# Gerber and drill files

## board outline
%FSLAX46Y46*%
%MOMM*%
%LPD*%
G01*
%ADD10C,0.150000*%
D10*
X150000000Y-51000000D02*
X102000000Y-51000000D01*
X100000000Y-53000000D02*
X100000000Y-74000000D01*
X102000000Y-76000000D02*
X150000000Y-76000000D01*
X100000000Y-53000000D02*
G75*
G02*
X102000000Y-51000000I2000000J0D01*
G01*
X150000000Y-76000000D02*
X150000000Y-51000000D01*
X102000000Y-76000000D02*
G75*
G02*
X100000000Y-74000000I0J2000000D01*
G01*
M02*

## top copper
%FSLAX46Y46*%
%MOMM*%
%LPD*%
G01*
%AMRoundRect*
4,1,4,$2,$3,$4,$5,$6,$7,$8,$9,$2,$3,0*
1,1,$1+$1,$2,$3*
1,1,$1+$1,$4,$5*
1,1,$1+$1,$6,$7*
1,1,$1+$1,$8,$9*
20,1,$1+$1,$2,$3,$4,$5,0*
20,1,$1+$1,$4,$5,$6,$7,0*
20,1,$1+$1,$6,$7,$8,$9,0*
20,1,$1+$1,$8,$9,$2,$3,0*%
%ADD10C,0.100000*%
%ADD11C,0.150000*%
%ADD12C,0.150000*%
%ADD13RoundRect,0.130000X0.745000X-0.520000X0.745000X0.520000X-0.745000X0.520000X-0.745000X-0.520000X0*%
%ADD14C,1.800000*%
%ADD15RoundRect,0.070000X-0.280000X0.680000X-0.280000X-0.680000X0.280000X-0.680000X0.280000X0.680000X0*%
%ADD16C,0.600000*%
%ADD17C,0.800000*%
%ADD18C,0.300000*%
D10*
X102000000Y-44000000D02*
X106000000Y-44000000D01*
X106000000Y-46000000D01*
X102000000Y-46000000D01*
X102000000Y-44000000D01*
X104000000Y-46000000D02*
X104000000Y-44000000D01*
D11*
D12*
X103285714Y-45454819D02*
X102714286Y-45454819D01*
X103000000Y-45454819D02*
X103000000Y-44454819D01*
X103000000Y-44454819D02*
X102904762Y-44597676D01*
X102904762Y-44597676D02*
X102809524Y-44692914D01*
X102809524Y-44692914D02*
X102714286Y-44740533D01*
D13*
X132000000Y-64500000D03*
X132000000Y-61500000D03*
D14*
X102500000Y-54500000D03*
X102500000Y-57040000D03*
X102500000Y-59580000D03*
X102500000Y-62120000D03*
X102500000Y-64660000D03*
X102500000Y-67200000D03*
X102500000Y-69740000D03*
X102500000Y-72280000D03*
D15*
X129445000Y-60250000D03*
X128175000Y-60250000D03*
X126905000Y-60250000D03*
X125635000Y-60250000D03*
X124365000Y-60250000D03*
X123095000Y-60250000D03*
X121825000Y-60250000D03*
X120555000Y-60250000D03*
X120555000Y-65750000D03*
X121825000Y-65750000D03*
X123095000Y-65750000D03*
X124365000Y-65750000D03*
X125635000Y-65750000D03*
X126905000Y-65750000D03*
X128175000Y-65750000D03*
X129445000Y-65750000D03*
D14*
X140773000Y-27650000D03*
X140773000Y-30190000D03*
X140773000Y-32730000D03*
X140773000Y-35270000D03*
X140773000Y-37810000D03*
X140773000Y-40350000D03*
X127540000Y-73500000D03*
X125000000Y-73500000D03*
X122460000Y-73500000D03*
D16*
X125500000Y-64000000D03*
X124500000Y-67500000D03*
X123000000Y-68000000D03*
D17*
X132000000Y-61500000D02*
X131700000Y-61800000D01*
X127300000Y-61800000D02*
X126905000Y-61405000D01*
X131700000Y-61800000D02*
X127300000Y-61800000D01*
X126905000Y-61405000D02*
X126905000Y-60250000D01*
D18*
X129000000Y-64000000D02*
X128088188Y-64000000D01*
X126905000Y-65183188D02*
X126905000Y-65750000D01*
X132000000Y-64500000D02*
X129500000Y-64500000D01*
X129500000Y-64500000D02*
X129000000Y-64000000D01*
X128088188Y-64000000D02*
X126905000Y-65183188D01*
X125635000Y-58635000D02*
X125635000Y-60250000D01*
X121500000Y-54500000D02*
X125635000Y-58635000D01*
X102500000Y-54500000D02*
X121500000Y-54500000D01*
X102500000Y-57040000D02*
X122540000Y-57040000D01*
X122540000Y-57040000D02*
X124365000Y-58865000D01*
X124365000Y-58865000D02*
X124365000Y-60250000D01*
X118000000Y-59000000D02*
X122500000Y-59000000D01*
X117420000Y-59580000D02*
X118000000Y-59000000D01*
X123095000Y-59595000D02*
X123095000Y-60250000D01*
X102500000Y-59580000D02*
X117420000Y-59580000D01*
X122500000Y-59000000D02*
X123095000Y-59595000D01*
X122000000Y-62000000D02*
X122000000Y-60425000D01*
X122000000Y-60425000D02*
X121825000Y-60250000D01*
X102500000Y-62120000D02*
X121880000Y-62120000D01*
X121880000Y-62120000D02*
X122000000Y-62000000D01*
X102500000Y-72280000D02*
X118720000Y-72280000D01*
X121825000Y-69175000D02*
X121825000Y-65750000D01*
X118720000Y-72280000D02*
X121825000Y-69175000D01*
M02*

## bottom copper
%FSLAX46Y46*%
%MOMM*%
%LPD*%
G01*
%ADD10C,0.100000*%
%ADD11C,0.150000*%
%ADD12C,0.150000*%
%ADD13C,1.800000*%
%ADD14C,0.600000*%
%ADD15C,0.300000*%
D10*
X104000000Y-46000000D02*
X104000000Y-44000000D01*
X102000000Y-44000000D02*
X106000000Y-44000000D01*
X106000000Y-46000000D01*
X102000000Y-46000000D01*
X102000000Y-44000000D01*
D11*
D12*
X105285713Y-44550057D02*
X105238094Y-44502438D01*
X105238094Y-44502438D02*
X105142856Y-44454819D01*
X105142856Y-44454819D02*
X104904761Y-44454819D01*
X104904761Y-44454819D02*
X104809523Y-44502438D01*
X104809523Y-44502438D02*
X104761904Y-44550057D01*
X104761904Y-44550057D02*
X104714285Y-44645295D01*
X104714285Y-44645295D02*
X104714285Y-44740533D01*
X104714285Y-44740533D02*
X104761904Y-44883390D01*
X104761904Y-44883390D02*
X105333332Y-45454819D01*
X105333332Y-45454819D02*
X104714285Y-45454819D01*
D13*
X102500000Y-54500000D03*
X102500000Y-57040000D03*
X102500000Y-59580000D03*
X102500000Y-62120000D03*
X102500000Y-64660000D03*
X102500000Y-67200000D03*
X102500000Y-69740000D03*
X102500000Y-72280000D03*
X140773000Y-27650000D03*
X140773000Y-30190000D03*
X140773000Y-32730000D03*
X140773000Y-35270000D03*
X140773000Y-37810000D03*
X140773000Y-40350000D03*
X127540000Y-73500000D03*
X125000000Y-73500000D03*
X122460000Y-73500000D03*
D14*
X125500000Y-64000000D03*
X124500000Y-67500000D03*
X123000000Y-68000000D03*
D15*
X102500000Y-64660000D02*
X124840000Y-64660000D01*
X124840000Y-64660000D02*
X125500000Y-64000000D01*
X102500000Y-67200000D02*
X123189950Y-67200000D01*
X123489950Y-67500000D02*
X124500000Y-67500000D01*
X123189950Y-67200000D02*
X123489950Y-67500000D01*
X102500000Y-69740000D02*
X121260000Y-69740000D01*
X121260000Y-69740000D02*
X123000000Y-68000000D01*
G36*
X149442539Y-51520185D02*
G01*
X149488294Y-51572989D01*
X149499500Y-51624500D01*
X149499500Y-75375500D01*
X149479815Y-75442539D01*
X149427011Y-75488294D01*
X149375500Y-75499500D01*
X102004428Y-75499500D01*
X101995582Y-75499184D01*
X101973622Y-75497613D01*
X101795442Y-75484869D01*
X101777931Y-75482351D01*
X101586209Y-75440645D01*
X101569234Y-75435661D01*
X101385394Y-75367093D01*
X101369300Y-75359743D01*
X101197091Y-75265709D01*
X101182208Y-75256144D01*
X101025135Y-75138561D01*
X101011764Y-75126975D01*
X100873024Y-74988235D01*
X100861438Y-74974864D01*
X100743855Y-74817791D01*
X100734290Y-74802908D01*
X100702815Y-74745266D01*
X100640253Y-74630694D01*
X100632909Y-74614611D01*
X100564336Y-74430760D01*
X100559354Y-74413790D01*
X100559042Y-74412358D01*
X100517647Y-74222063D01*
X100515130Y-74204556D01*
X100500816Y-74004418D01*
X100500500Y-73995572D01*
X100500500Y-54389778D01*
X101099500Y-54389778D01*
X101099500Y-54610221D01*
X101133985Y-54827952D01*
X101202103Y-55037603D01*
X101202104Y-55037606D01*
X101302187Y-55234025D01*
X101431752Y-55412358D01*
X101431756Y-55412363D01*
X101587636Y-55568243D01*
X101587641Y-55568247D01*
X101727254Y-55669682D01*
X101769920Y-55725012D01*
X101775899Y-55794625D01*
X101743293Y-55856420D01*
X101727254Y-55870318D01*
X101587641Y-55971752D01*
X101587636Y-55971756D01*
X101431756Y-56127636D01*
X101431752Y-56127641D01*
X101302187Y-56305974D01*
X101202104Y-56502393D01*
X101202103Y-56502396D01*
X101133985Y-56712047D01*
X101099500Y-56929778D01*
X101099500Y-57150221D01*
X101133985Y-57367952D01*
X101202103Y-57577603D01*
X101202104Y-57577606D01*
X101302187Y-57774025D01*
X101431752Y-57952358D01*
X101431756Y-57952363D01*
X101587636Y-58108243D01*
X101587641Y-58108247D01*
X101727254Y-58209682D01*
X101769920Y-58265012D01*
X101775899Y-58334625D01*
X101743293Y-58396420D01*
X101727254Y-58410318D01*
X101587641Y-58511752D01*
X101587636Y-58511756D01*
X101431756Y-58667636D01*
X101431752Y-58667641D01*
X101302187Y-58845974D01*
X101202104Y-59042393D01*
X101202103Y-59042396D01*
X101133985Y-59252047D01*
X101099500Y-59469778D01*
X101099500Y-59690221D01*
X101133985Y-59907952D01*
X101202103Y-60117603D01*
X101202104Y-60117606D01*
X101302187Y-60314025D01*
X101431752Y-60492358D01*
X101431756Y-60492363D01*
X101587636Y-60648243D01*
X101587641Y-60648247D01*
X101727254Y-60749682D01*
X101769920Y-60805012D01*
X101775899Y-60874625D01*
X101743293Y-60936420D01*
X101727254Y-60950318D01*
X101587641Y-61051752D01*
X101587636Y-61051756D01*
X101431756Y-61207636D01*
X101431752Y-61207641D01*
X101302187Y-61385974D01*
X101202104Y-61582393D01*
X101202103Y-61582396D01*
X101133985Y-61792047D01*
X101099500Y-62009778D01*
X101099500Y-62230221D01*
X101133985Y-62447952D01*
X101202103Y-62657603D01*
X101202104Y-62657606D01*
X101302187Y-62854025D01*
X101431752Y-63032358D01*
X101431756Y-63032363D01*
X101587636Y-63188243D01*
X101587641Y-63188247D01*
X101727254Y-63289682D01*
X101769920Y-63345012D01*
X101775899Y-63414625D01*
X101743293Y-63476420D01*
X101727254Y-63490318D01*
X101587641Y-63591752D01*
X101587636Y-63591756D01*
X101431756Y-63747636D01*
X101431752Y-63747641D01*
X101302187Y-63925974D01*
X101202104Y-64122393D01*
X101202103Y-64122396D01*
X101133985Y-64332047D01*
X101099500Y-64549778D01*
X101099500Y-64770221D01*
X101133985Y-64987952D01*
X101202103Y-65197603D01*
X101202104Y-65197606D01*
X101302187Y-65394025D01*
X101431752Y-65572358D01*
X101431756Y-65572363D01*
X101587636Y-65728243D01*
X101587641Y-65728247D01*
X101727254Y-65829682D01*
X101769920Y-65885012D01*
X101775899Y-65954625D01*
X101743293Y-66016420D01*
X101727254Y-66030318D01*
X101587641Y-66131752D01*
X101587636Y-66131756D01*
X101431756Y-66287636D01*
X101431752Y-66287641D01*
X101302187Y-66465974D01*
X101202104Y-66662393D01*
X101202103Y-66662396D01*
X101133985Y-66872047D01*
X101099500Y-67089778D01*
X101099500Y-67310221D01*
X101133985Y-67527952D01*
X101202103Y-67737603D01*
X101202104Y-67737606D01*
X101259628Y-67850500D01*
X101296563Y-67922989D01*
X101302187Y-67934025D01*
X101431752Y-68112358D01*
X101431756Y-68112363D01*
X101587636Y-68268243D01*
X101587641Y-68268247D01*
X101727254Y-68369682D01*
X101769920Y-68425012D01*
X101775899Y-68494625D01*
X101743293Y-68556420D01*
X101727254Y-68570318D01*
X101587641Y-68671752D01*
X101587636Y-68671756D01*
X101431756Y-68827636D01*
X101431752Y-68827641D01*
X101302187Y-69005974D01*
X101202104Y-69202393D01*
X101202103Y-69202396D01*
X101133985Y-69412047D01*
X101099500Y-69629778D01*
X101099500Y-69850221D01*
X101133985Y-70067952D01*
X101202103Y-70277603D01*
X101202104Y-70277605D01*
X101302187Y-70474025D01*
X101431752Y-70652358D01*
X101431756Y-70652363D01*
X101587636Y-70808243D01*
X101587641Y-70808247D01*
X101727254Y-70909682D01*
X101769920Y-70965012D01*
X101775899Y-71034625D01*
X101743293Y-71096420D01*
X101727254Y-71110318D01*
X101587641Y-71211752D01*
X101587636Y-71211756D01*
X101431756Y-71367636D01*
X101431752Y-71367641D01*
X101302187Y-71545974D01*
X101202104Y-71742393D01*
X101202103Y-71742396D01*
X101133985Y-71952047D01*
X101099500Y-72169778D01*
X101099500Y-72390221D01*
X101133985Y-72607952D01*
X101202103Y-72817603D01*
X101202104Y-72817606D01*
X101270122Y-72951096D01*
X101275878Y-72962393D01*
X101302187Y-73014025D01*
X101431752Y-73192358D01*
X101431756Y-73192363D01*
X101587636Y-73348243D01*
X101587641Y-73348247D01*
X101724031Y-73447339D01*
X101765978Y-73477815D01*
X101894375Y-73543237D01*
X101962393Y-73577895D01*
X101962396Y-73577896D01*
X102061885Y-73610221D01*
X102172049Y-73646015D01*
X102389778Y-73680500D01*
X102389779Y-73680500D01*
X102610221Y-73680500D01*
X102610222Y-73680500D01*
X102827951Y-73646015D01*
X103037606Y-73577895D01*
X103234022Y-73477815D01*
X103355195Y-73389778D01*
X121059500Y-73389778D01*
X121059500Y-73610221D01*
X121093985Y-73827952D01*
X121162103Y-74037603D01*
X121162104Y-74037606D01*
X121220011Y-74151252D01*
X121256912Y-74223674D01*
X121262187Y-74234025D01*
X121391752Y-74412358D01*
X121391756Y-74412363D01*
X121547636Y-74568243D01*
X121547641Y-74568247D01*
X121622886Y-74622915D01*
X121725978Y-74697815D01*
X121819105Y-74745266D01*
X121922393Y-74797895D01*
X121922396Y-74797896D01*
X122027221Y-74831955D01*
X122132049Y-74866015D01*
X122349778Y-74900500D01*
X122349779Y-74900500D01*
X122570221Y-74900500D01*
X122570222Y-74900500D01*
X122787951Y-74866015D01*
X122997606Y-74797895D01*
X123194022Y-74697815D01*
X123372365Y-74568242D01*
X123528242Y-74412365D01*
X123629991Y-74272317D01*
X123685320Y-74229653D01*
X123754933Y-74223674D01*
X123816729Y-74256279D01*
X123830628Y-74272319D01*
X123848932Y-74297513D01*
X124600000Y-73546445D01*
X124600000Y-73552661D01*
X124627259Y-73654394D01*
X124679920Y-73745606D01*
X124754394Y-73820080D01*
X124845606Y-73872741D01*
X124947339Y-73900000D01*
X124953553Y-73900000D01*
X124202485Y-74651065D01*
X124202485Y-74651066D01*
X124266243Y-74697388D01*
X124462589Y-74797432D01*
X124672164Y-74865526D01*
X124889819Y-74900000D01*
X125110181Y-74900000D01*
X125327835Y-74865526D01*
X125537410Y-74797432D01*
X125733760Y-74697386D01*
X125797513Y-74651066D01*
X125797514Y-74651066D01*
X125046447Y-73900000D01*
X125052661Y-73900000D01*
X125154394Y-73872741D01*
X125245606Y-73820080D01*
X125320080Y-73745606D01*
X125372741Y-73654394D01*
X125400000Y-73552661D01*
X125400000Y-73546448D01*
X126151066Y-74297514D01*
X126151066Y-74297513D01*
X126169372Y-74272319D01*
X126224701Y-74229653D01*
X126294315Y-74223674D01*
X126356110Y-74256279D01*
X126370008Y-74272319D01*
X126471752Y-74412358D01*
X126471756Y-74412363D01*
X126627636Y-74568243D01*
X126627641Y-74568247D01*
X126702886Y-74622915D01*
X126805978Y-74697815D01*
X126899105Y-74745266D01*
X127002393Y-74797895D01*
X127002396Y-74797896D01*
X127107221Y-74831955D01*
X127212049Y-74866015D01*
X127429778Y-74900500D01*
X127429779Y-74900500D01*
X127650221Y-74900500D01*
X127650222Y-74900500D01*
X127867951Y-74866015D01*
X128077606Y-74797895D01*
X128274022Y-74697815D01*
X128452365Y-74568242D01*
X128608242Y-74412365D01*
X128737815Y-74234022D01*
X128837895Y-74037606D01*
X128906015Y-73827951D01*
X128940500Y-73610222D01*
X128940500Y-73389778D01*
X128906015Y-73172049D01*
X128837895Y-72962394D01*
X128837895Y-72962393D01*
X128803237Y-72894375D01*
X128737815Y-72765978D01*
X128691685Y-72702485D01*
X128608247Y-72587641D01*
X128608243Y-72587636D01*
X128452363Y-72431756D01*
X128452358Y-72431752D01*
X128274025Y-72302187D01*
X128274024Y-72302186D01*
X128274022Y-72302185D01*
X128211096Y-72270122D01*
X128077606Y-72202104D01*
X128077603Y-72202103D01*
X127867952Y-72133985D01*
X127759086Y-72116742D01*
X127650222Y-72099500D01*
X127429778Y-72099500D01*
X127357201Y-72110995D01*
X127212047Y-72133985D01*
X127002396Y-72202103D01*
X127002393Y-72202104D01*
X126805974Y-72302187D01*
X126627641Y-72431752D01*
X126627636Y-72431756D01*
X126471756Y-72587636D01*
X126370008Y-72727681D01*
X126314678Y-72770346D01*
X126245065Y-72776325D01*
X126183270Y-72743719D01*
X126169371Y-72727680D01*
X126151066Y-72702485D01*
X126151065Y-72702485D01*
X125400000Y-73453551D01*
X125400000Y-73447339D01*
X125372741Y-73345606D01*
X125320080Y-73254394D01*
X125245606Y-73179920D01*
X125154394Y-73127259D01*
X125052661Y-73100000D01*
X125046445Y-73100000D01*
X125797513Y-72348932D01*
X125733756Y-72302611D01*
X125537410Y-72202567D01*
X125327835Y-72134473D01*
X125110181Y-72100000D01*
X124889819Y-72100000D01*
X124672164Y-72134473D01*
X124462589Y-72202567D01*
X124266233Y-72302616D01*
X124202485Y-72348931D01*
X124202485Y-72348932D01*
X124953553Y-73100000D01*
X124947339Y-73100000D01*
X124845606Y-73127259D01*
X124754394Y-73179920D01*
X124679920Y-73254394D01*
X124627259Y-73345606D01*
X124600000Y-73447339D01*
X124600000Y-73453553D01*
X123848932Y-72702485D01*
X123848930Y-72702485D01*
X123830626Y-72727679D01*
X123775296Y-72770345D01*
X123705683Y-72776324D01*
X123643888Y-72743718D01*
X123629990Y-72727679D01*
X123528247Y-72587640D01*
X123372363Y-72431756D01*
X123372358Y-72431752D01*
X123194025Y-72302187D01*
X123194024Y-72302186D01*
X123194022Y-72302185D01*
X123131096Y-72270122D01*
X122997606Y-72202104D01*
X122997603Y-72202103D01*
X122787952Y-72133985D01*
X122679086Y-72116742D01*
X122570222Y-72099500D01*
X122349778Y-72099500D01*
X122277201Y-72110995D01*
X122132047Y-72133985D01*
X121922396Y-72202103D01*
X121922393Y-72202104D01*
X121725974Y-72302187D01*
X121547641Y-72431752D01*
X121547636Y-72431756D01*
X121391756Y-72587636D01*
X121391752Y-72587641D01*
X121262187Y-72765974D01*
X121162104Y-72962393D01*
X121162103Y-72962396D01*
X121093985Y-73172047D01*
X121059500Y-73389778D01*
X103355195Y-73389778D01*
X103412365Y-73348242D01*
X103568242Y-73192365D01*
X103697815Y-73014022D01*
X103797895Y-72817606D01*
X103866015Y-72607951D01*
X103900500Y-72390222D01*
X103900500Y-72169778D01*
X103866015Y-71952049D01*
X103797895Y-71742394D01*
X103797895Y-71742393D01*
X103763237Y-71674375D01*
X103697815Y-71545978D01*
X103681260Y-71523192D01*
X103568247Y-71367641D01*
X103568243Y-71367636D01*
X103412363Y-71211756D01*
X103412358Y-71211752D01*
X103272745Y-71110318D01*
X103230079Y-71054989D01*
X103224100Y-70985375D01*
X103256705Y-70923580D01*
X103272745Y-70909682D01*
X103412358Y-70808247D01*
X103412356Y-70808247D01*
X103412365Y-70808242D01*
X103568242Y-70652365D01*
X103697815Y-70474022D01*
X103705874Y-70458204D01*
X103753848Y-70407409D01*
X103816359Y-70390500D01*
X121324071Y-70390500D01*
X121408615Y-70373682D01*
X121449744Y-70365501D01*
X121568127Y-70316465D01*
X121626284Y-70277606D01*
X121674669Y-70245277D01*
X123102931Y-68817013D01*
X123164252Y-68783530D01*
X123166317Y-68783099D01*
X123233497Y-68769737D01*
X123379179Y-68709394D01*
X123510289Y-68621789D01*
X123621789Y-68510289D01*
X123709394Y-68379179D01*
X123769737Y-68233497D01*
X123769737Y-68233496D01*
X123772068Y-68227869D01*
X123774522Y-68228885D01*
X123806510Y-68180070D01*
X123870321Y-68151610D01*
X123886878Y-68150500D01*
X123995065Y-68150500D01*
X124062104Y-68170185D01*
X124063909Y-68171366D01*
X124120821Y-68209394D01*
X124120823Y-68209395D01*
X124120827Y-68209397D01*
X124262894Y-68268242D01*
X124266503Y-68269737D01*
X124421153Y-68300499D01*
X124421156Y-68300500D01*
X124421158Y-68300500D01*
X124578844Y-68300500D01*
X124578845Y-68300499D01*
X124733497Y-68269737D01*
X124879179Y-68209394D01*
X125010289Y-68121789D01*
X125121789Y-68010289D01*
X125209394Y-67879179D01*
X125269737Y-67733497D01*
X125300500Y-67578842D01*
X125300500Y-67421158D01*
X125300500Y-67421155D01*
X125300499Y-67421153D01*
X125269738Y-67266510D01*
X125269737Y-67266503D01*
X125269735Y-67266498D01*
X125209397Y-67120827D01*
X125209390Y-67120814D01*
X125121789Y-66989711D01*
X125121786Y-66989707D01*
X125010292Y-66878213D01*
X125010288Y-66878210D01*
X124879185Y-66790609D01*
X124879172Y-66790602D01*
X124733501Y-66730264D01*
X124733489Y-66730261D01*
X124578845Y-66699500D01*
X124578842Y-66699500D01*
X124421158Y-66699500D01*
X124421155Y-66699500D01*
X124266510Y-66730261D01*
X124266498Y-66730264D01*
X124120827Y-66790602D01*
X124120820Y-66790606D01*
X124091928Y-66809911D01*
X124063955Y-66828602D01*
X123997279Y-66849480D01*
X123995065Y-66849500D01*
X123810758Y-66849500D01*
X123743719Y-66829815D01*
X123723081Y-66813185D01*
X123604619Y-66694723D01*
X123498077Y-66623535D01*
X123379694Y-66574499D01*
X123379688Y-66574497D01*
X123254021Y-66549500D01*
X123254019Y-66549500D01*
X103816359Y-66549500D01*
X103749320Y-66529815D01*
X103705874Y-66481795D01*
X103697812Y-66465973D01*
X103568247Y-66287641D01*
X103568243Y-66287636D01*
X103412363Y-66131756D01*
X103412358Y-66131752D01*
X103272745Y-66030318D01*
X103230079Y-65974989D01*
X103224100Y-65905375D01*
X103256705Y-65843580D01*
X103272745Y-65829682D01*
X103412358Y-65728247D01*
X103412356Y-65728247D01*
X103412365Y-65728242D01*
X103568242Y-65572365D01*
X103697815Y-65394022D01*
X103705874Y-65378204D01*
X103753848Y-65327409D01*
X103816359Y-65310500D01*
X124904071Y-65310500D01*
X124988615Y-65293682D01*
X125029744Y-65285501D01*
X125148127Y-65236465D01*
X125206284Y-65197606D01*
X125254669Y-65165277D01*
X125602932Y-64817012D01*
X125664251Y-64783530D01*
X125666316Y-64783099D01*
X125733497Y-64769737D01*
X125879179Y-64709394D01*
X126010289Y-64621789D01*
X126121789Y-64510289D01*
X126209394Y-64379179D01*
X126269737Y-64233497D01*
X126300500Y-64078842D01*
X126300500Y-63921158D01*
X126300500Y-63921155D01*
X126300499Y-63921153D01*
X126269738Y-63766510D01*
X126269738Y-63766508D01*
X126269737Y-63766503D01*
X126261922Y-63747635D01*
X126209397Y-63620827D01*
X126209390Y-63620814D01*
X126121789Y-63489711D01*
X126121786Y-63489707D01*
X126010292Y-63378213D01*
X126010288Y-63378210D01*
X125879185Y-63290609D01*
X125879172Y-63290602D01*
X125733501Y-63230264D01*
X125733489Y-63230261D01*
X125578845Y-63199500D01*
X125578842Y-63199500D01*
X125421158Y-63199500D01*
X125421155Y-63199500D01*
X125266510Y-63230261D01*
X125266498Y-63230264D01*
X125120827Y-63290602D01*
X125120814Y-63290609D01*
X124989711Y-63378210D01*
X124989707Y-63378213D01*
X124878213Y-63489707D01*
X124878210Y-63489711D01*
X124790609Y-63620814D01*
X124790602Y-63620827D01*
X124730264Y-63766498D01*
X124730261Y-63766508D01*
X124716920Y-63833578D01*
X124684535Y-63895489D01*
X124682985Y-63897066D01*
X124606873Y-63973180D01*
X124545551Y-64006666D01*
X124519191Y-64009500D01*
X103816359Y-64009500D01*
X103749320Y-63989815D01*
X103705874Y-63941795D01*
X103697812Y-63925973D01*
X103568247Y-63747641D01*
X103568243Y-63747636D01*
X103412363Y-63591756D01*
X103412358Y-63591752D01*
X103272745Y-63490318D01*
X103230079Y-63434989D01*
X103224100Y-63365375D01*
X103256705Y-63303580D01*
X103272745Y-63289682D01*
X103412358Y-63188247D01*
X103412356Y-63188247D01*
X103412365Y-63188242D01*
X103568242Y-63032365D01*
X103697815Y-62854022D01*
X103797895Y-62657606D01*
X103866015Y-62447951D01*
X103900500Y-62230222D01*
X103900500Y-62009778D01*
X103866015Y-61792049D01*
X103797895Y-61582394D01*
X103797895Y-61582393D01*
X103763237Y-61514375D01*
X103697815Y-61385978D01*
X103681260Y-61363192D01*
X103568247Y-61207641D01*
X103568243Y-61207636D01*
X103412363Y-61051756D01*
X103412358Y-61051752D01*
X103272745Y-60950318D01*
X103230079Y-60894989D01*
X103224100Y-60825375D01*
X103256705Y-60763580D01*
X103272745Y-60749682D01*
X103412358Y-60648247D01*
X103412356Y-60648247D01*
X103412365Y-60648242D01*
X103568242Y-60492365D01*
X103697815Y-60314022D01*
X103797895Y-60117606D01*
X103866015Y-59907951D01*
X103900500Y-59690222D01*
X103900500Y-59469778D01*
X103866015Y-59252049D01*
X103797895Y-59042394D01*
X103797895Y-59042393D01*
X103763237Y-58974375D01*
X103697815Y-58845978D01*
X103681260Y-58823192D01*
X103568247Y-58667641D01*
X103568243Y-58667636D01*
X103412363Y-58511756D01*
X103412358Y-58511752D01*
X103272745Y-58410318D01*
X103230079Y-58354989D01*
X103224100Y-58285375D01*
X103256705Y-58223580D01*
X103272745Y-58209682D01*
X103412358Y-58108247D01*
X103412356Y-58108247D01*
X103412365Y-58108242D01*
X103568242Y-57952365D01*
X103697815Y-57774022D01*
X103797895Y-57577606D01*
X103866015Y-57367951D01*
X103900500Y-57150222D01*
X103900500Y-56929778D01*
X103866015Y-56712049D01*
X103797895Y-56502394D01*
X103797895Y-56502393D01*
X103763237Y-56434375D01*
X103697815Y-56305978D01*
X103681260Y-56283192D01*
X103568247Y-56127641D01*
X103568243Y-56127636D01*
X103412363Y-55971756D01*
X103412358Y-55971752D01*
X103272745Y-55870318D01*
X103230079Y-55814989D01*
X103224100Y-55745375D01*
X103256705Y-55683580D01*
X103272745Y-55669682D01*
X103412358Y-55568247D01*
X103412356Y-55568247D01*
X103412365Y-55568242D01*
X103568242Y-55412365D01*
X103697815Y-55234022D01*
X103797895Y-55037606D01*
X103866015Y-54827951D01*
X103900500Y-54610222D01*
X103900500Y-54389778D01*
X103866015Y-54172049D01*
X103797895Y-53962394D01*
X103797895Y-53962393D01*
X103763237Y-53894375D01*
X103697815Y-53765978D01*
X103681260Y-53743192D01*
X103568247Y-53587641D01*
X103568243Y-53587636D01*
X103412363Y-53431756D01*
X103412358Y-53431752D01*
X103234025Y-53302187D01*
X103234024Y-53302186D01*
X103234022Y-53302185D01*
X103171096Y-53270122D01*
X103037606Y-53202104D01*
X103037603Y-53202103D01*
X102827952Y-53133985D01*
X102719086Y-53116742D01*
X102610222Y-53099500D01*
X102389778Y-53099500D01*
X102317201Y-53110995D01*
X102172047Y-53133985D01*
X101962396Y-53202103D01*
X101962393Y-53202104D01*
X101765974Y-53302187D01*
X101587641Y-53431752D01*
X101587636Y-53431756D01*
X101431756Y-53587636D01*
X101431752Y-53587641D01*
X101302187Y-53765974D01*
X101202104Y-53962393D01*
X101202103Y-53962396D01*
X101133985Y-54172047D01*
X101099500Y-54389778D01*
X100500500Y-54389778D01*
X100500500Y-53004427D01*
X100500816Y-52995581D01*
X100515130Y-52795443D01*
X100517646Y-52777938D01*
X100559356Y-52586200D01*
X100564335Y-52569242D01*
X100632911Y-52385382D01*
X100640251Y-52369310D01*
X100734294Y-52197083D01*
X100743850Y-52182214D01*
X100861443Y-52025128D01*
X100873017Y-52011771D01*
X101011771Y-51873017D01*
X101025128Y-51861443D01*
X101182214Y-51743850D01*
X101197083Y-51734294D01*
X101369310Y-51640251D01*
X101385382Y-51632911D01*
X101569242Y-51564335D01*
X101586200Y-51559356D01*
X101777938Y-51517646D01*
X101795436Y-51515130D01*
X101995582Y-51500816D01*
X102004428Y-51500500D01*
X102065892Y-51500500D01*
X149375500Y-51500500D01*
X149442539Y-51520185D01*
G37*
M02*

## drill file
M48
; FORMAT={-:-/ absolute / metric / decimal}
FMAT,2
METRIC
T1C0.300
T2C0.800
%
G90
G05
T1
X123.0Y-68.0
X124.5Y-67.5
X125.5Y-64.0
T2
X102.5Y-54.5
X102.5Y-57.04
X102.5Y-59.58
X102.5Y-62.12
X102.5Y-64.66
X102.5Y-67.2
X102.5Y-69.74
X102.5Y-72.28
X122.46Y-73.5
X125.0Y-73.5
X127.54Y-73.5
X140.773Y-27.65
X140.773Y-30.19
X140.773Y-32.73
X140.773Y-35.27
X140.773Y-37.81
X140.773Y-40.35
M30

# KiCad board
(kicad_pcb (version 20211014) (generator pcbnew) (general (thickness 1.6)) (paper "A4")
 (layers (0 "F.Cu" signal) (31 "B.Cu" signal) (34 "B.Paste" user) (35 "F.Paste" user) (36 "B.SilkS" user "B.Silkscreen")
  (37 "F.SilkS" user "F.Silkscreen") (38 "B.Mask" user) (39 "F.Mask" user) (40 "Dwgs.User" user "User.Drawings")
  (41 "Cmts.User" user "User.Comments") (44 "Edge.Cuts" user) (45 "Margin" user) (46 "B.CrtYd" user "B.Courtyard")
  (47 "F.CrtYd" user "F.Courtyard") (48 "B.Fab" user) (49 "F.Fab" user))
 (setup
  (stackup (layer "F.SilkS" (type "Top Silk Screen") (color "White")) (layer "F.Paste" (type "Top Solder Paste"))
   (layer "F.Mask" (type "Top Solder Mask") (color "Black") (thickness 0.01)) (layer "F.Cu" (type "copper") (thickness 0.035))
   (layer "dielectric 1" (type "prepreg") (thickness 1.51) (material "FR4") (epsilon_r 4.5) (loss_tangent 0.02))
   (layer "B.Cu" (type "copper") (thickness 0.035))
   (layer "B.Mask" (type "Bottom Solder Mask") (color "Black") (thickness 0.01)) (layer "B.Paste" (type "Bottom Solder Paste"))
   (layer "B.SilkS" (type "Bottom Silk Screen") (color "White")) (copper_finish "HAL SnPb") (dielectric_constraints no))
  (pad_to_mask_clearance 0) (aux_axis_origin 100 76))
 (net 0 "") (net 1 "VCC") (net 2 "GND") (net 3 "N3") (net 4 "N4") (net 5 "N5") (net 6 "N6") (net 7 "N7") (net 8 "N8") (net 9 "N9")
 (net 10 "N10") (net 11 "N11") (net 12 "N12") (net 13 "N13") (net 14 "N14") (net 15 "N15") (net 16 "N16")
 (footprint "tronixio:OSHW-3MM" (layer "F.Cu") (at 148 73.5)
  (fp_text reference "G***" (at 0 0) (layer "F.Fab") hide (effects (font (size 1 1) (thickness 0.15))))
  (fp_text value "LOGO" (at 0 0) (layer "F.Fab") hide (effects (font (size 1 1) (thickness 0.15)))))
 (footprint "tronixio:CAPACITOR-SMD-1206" (layer "F.Cu") (at 132 63 90) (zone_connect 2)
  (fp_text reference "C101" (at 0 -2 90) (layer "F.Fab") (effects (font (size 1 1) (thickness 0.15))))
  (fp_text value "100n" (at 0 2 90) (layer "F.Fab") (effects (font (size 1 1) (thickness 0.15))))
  (pad "1" smd roundrect (at -1.5 0 90) (size 1.3 1.75) (layers "F.Cu" "F.Paste" "F.Mask") (roundrect_rratio 0.1) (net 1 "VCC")
   (zone_connect 2))
  (pad "2" smd roundrect (at 1.5 0 90) (size 1.3 1.75) (layers "F.Cu" "F.Paste" "F.Mask") (roundrect_rratio 0.1) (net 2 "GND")
   (zone_connect 2)))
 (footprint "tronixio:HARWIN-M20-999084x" (layer "F.Cu") (at 102.5 54.5)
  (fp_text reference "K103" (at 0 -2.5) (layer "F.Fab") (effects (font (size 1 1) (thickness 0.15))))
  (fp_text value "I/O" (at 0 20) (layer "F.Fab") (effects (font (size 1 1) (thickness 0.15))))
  (pad "1" thru_hole circle locked (at 0 0) (size 1.8 1.8) (drill 0.8) (layers *.Cu *.Mask) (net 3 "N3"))
  (pad "2" thru_hole circle (at 0 2.54) (size 1.8 1.8) (drill 0.8) (layers *.Cu *.Mask) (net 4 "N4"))
  (pad "3" thru_hole circle (at 0 5.08) (size 1.8 1.8) (drill 0.8) (layers *.Cu *.Mask) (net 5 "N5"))
  (pad "4" thru_hole circle (at 0 7.62) (size 1.8 1.8) (drill 0.8) (layers *.Cu *.Mask) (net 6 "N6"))
  (pad "5" thru_hole circle (at 0 10.16) (size 1.8 1.8) (drill 0.8) (layers *.Cu *.Mask) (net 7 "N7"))
  (pad "6" thru_hole circle (at 0 12.7) (size 1.8 1.8) (drill 0.8) (layers *.Cu *.Mask) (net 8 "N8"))
  (pad "7" thru_hole circle (at 0 15.24) (size 1.8 1.8) (drill 0.8) (layers *.Cu *.Mask) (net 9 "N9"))
  (pad "8" thru_hole circle (at 0 17.78) (size 1.8 1.8) (drill 0.8) (layers *.Cu *.Mask) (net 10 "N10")))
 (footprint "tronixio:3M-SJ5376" (layer "F.Cu") (at 166.4 61.25)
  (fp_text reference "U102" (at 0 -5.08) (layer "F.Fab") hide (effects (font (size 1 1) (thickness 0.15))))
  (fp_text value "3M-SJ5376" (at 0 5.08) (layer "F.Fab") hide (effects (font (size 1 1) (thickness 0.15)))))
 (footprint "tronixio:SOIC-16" (layer "F.Cu") (at 125 63 -90)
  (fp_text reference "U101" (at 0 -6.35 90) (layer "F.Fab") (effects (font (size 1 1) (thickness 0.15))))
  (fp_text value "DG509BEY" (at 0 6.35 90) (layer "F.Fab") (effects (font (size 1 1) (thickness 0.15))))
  (pad "1" smd roundrect (at -2.75 -4.445 270) (size 1.5 0.7) (layers "F.Cu" "F.Paste" "F.Mask") (roundrect_rratio 0.1) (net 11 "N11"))
  (pad "2" smd roundrect (at -2.75 -3.175 270) (size 1.5 0.7) (layers "F.Cu" "F.Paste" "F.Mask") (roundrect_rratio 0.1) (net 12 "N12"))
  (pad "3" smd roundrect (at -2.75 -1.905 270) (size 1.5 0.7) (layers "F.Cu" "F.Paste" "F.Mask") (roundrect_rratio 0.1) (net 2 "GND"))
  (pad "4" smd roundrect (at -2.75 -0.635 270) (size 1.5 0.7) (layers "F.Cu" "F.Paste" "F.Mask") (roundrect_rratio 0.1) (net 3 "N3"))
  (pad "5" smd roundrect (at -2.75 0.635 270) (size 1.5 0.7) (layers "F.Cu" "F.Paste" "F.Mask") (roundrect_rratio 0.1) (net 4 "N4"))
  (pad "6" smd roundrect (at -2.75 1.905 270) (size 1.5 0.7) (layers "F.Cu" "F.Paste" "F.Mask") (roundrect_rratio 0.1) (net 5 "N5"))
  (pad "7" smd roundrect (at -2.75 3.175 270) (size 1.5 0.7) (layers "F.Cu" "F.Paste" "F.Mask") (roundrect_rratio 0.1) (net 6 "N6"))
  (pad "8" smd roundrect (at -2.75 4.445 270) (size 1.5 0.7) (layers "F.Cu" "F.Paste" "F.Mask") (roundrect_rratio 0.1) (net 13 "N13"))
  (pad "9" smd roundrect (at 2.75 4.445 270) (size 1.5 0.7) (layers "F.Cu" "F.Paste" "F.Mask") (roundrect_rratio 0.1) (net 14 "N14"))
  (pad "10" smd roundrect (at 2.75 3.175 270) (size 1.5 0.7) (layers "F.Cu" "F.Paste" "F.Mask") (roundrect_rratio 0.1) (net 10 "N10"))
  (pad "11" smd roundrect (at 2.75 1.905 270) (size 1.5 0.7) (layers "F.Cu" "F.Paste" "F.Mask") (roundrect_rratio 0.1) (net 9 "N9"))
  (pad "12" smd roundrect (at 2.75 0.635 270) (size 1.5 0.7) (layers "F.Cu" "F.Paste" "F.Mask") (roundrect_rratio 0.1) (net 8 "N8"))
  (pad "13" smd roundrect (at 2.75 -0.635 270) (size 1.5 0.7) (layers "F.Cu" "F.Paste" "F.Mask") (roundrect_rratio 0.1) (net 7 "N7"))
  (pad "14" smd roundrect (at 2.75 -1.905 270) (size 1.5 0.7) (layers "F.Cu" "F.Paste" "F.Mask") (roundrect_rratio 0.1) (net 1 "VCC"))
  (pad "15" smd roundrect (at 2.75 -3.175 270) (size 1.5 0.7) (layers "F.Cu" "F.Paste" "F.Mask") (roundrect_rratio 0.1) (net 2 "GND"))
  (pad "16" smd roundrect (at 2.75 -4.445 270) (size 1.5 0.7) (layers "F.Cu" "F.Paste" "F.Mask") (roundrect_rratio 0.1) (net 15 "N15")))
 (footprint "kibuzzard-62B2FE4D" (layer "F.Cu") (at 142.25 59.69)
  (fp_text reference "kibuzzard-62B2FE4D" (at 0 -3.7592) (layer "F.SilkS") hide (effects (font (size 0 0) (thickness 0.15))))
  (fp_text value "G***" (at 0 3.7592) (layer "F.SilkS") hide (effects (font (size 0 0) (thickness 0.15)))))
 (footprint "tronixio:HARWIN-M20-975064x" (layer "F.Cu") (at 140.773 27.65 -90)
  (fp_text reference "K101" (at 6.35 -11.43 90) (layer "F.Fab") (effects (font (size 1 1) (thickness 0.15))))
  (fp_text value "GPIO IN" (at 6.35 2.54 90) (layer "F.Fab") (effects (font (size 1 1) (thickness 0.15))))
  (pad "1" thru_hole circle (at 0 0 270) (size 1.8 1.8) (drill 0.8) (layers *.Cu *.Mask) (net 1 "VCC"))
  (pad "2" thru_hole circle (at 2.54 0 270) (size 1.8 1.8) (drill 0.8) (layers *.Cu *.Mask) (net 2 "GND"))
  (pad "3" thru_hole circle (at 5.08 0 270) (size 1.8 1.8) (drill 0.8) (layers *.Cu *.Mask) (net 12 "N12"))
  (pad "4" thru_hole circle (at 7.62 0 270) (size 1.8 1.8) (drill 0.8) (layers *.Cu *.Mask) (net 11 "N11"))
  (pad "5" thru_hole circle (at 10.16 0 270) (size 1.8 1.8) (drill 0.8) (layers *.Cu *.Mask) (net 15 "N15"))
  (pad "6" thru_hole circle (at 12.7 0 270) (size 1.8 1.8) (drill 0.8) (layers *.Cu *.Mask) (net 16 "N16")))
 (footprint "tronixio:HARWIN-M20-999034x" (layer "F.Cu") (at 127.54 73.5 -90)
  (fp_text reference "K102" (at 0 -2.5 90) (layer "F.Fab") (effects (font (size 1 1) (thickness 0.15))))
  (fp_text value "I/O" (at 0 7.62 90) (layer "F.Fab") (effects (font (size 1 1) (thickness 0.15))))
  (pad "1" thru_hole circle locked (at 0 0 270) (size 1.8 1.8) (drill 0.8) (layers *.Cu *.Mask) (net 13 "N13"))
  (pad "2" thru_hole circle (at 0 2.54 270) (size 1.8 1.8) (drill 0.8) (layers *.Cu *.Mask) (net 2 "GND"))
  (pad "3" thru_hole circle (at 0 5.08 270) (size 1.8 1.8) (drill 0.8) (layers *.Cu *.Mask) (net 14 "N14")))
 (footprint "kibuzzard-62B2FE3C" (layer "F.Cu") (at 142.25 57.15)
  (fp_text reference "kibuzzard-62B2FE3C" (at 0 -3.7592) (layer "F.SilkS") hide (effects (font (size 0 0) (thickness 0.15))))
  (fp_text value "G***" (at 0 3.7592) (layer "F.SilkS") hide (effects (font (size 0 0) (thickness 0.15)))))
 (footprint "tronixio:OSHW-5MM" (layer "B.Cu") (at 125 57 180)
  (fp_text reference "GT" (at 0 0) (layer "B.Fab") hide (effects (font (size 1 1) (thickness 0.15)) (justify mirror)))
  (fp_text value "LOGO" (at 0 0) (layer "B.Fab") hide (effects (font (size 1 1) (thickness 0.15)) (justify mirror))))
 (gr_rect (start 102 46) (end 106 44) (layer "F.Cu") (width 0.1) (fill none))
 (gr_line (start 104 46) (end 104 44) (layer "F.Cu") (width 0.1))
 (gr_line (start 104 46) (end 104 44) (layer "B.Cu") (width 0.1))
 (gr_rect (start 102 46) (end 106 44) (layer "B.Cu") (width 0.1) (fill none))
 (gr_line (start 150 51) (end 102 51) (layer "Edge.Cuts") (width 0.15))
 (gr_line (start 100 53) (end 100 74) (layer "Edge.Cuts") (width 0.15))
 (gr_line (start 102 76) (end 150 76) (layer "Edge.Cuts") (width 0.15))
 (gr_arc (start 100 53) (mid 100.585786 51.585786) (end 102 51) (layer "Edge.Cuts") (width 0.15))
 (gr_line (start 150 76) (end 150 51) (layer "Edge.Cuts") (width 0.15))
 (gr_arc (start 102 76) (mid 100.585786 75.414214) (end 100 74) (layer "Edge.Cuts") (width 0.15))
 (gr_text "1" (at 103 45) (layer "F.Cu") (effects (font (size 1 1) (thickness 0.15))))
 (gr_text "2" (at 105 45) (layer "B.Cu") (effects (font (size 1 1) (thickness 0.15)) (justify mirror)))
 (segment (start 132 61.5) (end 131.7 61.8) (width 0.8) (layer "F.Cu") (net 2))
 (segment (start 127.3 61.8) (end 126.905 61.405) (width 0.8) (layer "F.Cu") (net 2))
 (segment (start 131.7 61.8) (end 127.3 61.8) (width 0.8) (layer "F.Cu") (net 2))
 (segment (start 126.905 61.405) (end 126.905 60.25) (width 0.8) (layer "F.Cu") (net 2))
 (segment (start 129 64) (end 128.088188 64) (width 0.3) (layer "F.Cu") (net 1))
 (segment (start 126.905 65.183188) (end 126.905 65.75) (width 0.3) (layer "F.Cu") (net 1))
 (segment (start 132 64.5) (end 129.5 64.5) (width 0.3) (layer "F.Cu") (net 1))
 (segment (start 129.5 64.5) (end 129 64) (width 0.3) (layer "F.Cu") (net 1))
 (segment (start 128.088188 64) (end 126.905 65.183188) (width 0.3) (layer "F.Cu") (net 1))
 (segment (start 125.635 58.635) (end 125.635 60.25) (width 0.3) (layer "F.Cu") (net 3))
 (segment (start 121.5 54.5) (end 125.635 58.635) (width 0.3) (layer "F.Cu") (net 3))
 (segment (start 102.5 54.5) (end 121.5 54.5) (width 0.3) (layer "F.Cu") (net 3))
 (segment (start 102.5 57.04) (end 122.54 57.04) (width 0.3) (layer "F.Cu") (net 4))
 (segment (start 122.54 57.04) (end 124.365 58.865) (width 0.3) (layer "F.Cu") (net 4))
 (segment (start 124.365 58.865) (end 124.365 60.25) (width 0.3) (layer "F.Cu") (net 4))
 (segment (start 118 59) (end 122.5 59) (width 0.3) (layer "F.Cu") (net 5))
 (segment (start 117.42 59.58) (end 118 59) (width 0.3) (layer "F.Cu") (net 5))
 (segment (start 123.095 59.595) (end 123.095 60.25) (width 0.3) (layer "F.Cu") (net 5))
 (segment (start 102.5 59.58) (end 117.42 59.58) (width 0.3) (layer "F.Cu") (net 5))
 (segment (start 122.5 59) (end 123.095 59.595) (width 0.3) (layer "F.Cu") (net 5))
 (segment (start 122 62) (end 122 60.425) (width 0.3) (layer "F.Cu") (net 6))
 (segment (start 122 60.425) (end 121.825 60.25) (width 0.3) (layer "F.Cu") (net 6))
 (segment (start 102.5 62.12) (end 121.88 62.12) (width 0.3) (layer "F.Cu") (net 6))
 (segment (start 121.88 62.12) (end 122 62) (width 0.3) (layer "F.Cu") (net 6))
 (via (at 125.5 64) (size 0.6) (drill 0.3) (layers "F.Cu" "B.Cu") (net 7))
 (segment (start 102.5 64.66) (end 124.84 64.66) (width 0.3) (layer "B.Cu") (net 7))
 (segment (start 124.84 64.66) (end 125.5 64) (width 0.3) (layer "B.Cu") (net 7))
 (via (at 124.5 67.5) (size 0.6) (drill 0.3) (layers "F.Cu" "B.Cu") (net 8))
 (segment (start 102.5 67.2) (end 123.18995 67.2) (width 0.3) (layer "B.Cu") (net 8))
 (segment (start 123.48995 67.5) (end 124.5 67.5) (width 0.3) (layer "B.Cu") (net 8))
 (segment (start 123.18995 67.2) (end 123.48995 67.5) (width 0.3) (layer "B.Cu") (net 8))
 (via (at 123 68) (size 0.6) (drill 0.3) (layers "F.Cu" "B.Cu") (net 9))
 (segment (start 102.5 69.74) (end 121.26 69.74) (width 0.3) (layer "B.Cu") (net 9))
 (segment (start 121.26 69.74) (end 123 68) (width 0.3) (layer "B.Cu") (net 9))
 (segment (start 102.5 72.28) (end 118.72 72.28) (width 0.3) (layer "F.Cu") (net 10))
 (segment (start 121.825 69.175) (end 121.825 65.75) (width 0.3) (layer "F.Cu") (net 10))
 (segment (start 118.72 72.28) (end 121.825 69.175) (width 0.3) (layer "F.Cu") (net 10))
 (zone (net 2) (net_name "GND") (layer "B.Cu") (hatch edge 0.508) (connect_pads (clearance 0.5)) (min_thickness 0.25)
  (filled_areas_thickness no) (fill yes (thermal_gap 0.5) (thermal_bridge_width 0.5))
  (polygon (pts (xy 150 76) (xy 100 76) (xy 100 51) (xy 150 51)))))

